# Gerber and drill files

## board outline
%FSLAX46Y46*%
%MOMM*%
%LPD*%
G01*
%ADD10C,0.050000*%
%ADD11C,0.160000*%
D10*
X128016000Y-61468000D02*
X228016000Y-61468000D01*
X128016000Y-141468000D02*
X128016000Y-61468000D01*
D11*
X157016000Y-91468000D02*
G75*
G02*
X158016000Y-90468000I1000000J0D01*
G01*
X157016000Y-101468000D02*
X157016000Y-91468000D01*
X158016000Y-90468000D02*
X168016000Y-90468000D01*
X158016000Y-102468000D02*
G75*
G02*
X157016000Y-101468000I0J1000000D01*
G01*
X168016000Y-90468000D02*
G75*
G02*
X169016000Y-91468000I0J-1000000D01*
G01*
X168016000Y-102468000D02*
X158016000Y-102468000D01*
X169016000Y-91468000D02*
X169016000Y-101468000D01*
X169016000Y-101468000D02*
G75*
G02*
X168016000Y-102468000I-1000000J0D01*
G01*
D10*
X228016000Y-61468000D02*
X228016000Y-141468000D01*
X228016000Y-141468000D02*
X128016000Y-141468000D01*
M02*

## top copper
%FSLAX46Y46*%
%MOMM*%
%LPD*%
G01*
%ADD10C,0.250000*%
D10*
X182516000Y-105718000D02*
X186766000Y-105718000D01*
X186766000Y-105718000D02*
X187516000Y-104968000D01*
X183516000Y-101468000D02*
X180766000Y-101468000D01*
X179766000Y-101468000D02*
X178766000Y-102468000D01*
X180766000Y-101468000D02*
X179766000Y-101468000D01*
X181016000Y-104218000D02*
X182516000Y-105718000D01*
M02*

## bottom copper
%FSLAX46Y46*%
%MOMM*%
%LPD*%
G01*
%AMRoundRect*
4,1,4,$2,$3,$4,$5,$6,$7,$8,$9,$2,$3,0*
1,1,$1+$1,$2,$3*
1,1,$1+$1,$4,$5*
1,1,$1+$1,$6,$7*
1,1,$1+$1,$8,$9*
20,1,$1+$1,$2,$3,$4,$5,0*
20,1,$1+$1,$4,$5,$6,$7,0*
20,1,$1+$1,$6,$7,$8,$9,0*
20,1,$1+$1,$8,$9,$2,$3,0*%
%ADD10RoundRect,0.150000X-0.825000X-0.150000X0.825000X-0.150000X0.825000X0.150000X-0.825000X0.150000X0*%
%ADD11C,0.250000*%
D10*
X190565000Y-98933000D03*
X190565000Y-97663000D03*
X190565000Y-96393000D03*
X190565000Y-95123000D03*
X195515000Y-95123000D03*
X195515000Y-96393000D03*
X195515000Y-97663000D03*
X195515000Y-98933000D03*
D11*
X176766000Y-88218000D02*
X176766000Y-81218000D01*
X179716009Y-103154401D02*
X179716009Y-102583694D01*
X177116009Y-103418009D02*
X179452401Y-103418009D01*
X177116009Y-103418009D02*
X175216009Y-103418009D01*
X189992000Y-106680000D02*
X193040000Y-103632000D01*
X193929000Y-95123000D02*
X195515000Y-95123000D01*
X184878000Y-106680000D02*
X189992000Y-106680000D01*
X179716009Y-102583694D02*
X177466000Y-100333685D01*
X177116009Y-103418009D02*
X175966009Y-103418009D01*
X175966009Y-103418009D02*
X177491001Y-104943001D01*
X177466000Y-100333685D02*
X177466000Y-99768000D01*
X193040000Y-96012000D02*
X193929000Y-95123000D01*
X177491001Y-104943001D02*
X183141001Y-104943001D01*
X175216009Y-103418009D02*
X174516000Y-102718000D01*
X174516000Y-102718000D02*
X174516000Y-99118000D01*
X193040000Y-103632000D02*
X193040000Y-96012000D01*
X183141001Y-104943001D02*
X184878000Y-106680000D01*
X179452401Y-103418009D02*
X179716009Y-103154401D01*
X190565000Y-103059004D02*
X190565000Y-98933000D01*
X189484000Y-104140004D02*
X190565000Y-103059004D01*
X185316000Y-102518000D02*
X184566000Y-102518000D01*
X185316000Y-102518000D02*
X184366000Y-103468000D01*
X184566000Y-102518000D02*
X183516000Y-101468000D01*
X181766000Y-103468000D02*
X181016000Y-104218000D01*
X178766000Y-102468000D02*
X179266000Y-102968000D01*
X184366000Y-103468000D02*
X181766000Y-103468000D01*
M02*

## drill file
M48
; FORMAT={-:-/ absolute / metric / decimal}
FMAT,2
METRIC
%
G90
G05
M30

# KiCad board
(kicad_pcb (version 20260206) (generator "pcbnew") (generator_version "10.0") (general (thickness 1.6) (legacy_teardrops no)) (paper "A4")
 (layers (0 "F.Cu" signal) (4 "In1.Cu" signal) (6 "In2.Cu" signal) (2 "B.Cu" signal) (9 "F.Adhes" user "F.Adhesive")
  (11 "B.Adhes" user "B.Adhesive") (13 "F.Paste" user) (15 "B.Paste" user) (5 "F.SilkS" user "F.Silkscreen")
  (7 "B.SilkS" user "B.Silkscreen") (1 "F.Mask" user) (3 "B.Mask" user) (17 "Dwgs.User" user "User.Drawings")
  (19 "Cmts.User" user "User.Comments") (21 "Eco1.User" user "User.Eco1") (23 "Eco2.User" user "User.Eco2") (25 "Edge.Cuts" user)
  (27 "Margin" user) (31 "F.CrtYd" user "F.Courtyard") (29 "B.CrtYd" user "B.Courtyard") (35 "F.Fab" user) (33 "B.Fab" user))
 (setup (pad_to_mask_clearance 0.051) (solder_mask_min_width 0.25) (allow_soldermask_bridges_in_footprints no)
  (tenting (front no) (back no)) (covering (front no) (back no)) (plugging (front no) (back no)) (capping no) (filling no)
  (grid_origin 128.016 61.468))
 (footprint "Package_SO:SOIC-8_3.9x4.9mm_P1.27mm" (layer "B.Cu") (at 193.04 97.028)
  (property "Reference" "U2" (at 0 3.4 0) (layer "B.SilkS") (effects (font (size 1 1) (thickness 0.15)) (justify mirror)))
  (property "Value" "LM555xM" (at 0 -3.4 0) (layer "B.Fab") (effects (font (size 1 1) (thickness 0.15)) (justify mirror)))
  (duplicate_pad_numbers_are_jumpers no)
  (pad "1" smd roundrect (at -2.475 1.905) (size 1.95 0.6) (layers "B.Cu" "B.Mask" "B.Paste") (roundrect_rratio 0.25) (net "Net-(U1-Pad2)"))
  (pad "2" smd roundrect (at -2.475 0.635) (size 1.95 0.6) (layers "B.Cu" "B.Mask" "B.Paste") (roundrect_rratio 0.25) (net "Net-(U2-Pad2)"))
  (pad "3" smd roundrect (at -2.475 -0.635) (size 1.95 0.6) (layers "B.Cu" "B.Mask" "B.Paste") (roundrect_rratio 0.25) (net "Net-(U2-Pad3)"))
  (pad "4" smd roundrect (at -2.475 -1.905) (size 1.95 0.6) (layers "B.Cu" "B.Mask" "B.Paste") (roundrect_rratio 0.25) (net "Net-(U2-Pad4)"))
  (pad "5" smd roundrect (at 2.475 -1.905) (size 1.95 0.6) (layers "B.Cu" "B.Mask" "B.Paste") (roundrect_rratio 0.25) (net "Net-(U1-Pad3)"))
  (pad "6" smd roundrect (at 2.475 -0.635) (size 1.95 0.6) (layers "B.Cu" "B.Mask" "B.Paste") (roundrect_rratio 0.25) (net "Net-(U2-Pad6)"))
  (pad "7" smd roundrect (at 2.475 0.635) (size 1.95 0.6) (layers "B.Cu" "B.Mask" "B.Paste") (roundrect_rratio 0.25) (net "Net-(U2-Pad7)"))
  (pad "8" smd roundrect (at 2.475 1.905) (size 1.95 0.6) (layers "B.Cu" "B.Mask" "B.Paste") (roundrect_rratio 0.25) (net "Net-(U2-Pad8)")))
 (gr_line (start 128.016 61.468) (end 228.016 61.468) (stroke (width 0.05) (type solid)) (layer "Edge.Cuts"))
 (gr_line (start 128.016 141.468) (end 128.016 61.468) (stroke (width 0.05) (type solid)) (layer "Edge.Cuts"))
 (gr_arc (start 157.016 91.468) (mid 157.308893 90.760893) (end 158.016 90.468) (stroke (width 0.16) (type solid)) (layer "Edge.Cuts"))
 (gr_line (start 157.016 101.468) (end 157.016 91.468) (stroke (width 0.16) (type solid)) (layer "Edge.Cuts"))
 (gr_line (start 158.016 90.468) (end 168.016 90.468) (stroke (width 0.16) (type solid)) (layer "Edge.Cuts"))
 (gr_arc (start 158.016 102.468) (mid 157.308893 102.175107) (end 157.016 101.468) (stroke (width 0.16) (type solid)) (layer "Edge.Cuts"))
 (gr_arc (start 168.016 90.468) (mid 168.723107 90.760893) (end 169.016 91.468) (stroke (width 0.16) (type solid)) (layer "Edge.Cuts"))
 (gr_line (start 168.016 102.468) (end 158.016 102.468) (stroke (width 0.16) (type solid)) (layer "Edge.Cuts"))
 (gr_line (start 169.016 91.468) (end 169.016 101.468) (stroke (width 0.16) (type solid)) (layer "Edge.Cuts"))
 (gr_arc (start 169.016 101.468) (mid 168.723107 102.175107) (end 168.016 102.468) (stroke (width 0.16) (type solid)) (layer "Edge.Cuts"))
 (gr_line (start 228.016 61.468) (end 228.016 141.468) (stroke (width 0.05) (type solid)) (layer "Edge.Cuts"))
 (gr_line (start 228.016 141.468) (end 128.016 141.468) (stroke (width 0.05) (type solid)) (layer "Edge.Cuts"))
 (segment (start 176.766 88.218) (end 176.766 81.218) (width 0.25) (layer "B.Cu") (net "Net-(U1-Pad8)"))
 (segment (start 179.716009 103.154401) (end 179.716009 102.583694) (width 0.25) (layer "B.Cu") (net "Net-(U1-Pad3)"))
 (segment (start 177.116009 103.418009) (end 179.452401 103.418009) (width 0.25) (layer "B.Cu") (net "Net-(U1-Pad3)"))
 (segment (start 177.116009 103.418009) (end 175.216009 103.418009) (width 0.25) (layer "B.Cu") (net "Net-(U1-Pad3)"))
 (segment (start 189.992 106.68) (end 193.04 103.632) (width 0.25) (layer "B.Cu") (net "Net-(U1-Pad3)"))
 (segment (start 193.929 95.123) (end 195.515 95.123) (width 0.25) (layer "B.Cu") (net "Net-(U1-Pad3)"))
 (segment (start 184.878 106.68) (end 189.992 106.68) (width 0.25) (layer "B.Cu") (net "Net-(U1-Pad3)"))
 (segment (start 179.716009 102.583694) (end 177.466 100.333685) (width 0.25) (layer "B.Cu") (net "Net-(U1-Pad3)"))
 (segment (start 177.116009 103.418009) (end 175.966009 103.418009) (width 0.25) (layer "B.Cu") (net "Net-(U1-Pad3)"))
 (segment (start 175.966009 103.418009) (end 177.491001 104.943001) (width 0.25) (layer "B.Cu") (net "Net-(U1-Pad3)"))
 (segment (start 177.466 100.333685) (end 177.466 99.768) (width 0.25) (layer "B.Cu") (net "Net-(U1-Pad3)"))
 (segment (start 193.04 96.012) (end 193.929 95.123) (width 0.25) (layer "B.Cu") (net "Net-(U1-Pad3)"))
 (segment (start 177.491001 104.943001) (end 183.141001 104.943001) (width 0.25) (layer "B.Cu") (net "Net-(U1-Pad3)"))
 (segment (start 175.216009 103.418009) (end 174.516 102.718) (width 0.25) (layer "B.Cu") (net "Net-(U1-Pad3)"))
 (segment (start 174.516 102.718) (end 174.516 99.118) (width 0.25) (layer "B.Cu") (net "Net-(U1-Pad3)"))
 (segment (start 193.04 103.632) (end 193.04 96.012) (width 0.25) (layer "B.Cu") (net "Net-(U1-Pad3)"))
 (segment (start 183.141001 104.943001) (end 184.878 106.68) (width 0.25) (layer "B.Cu") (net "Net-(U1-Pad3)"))
 (segment (start 179.452401 103.418009) (end 179.716009 103.154401) (width 0.25) (layer "B.Cu") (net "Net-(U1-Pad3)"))
 (segment (start 190.565 103.059004) (end 190.565 98.933) (width 0.25) (layer "B.Cu") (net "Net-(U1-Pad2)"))
 (segment (start 189.484 104.140004) (end 190.565 103.059004) (width 0.25) (layer "B.Cu") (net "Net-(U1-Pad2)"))
 (segment (start 182.516 105.718) (end 186.766 105.718) (width 0.25) (layer "F.Cu") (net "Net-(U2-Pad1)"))
 (segment (start 186.766 105.718) (end 187.516 104.968) (width 0.25) (layer "F.Cu") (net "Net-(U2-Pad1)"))
 (segment (start 183.516 101.468) (end 180.766 101.468) (width 0.25) (layer "F.Cu") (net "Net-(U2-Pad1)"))
 (segment (start 179.766 101.468) (end 178.766 102.468) (width 0.25) (layer "F.Cu") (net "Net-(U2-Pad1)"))
 (segment (start 180.766 101.468) (end 179.766 101.468) (width 0.25) (layer "F.Cu") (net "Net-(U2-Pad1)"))
 (segment (start 181.016 104.218) (end 182.516 105.718) (width 0.25) (layer "F.Cu") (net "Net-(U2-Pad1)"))
 (segment (start 185.316 102.518) (end 184.566 102.518) (width 0.25) (layer "B.Cu") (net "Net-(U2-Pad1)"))
 (segment (start 185.316 102.518) (end 184.366 103.468) (width 0.25) (layer "B.Cu") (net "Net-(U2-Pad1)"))
 (segment (start 184.566 102.518) (end 183.516 101.468) (width 0.25) (layer "B.Cu") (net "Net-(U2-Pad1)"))
 (segment (start 181.766 103.468) (end 181.016 104.218) (width 0.25) (layer "B.Cu") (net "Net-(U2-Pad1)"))
 (segment (start 178.766 102.468) (end 179.266 102.968) (width 0.25) (layer "B.Cu") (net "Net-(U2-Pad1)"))
 (segment (start 184.366 103.468) (end 181.766 103.468) (width 0.25) (layer "B.Cu") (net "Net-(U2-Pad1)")))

